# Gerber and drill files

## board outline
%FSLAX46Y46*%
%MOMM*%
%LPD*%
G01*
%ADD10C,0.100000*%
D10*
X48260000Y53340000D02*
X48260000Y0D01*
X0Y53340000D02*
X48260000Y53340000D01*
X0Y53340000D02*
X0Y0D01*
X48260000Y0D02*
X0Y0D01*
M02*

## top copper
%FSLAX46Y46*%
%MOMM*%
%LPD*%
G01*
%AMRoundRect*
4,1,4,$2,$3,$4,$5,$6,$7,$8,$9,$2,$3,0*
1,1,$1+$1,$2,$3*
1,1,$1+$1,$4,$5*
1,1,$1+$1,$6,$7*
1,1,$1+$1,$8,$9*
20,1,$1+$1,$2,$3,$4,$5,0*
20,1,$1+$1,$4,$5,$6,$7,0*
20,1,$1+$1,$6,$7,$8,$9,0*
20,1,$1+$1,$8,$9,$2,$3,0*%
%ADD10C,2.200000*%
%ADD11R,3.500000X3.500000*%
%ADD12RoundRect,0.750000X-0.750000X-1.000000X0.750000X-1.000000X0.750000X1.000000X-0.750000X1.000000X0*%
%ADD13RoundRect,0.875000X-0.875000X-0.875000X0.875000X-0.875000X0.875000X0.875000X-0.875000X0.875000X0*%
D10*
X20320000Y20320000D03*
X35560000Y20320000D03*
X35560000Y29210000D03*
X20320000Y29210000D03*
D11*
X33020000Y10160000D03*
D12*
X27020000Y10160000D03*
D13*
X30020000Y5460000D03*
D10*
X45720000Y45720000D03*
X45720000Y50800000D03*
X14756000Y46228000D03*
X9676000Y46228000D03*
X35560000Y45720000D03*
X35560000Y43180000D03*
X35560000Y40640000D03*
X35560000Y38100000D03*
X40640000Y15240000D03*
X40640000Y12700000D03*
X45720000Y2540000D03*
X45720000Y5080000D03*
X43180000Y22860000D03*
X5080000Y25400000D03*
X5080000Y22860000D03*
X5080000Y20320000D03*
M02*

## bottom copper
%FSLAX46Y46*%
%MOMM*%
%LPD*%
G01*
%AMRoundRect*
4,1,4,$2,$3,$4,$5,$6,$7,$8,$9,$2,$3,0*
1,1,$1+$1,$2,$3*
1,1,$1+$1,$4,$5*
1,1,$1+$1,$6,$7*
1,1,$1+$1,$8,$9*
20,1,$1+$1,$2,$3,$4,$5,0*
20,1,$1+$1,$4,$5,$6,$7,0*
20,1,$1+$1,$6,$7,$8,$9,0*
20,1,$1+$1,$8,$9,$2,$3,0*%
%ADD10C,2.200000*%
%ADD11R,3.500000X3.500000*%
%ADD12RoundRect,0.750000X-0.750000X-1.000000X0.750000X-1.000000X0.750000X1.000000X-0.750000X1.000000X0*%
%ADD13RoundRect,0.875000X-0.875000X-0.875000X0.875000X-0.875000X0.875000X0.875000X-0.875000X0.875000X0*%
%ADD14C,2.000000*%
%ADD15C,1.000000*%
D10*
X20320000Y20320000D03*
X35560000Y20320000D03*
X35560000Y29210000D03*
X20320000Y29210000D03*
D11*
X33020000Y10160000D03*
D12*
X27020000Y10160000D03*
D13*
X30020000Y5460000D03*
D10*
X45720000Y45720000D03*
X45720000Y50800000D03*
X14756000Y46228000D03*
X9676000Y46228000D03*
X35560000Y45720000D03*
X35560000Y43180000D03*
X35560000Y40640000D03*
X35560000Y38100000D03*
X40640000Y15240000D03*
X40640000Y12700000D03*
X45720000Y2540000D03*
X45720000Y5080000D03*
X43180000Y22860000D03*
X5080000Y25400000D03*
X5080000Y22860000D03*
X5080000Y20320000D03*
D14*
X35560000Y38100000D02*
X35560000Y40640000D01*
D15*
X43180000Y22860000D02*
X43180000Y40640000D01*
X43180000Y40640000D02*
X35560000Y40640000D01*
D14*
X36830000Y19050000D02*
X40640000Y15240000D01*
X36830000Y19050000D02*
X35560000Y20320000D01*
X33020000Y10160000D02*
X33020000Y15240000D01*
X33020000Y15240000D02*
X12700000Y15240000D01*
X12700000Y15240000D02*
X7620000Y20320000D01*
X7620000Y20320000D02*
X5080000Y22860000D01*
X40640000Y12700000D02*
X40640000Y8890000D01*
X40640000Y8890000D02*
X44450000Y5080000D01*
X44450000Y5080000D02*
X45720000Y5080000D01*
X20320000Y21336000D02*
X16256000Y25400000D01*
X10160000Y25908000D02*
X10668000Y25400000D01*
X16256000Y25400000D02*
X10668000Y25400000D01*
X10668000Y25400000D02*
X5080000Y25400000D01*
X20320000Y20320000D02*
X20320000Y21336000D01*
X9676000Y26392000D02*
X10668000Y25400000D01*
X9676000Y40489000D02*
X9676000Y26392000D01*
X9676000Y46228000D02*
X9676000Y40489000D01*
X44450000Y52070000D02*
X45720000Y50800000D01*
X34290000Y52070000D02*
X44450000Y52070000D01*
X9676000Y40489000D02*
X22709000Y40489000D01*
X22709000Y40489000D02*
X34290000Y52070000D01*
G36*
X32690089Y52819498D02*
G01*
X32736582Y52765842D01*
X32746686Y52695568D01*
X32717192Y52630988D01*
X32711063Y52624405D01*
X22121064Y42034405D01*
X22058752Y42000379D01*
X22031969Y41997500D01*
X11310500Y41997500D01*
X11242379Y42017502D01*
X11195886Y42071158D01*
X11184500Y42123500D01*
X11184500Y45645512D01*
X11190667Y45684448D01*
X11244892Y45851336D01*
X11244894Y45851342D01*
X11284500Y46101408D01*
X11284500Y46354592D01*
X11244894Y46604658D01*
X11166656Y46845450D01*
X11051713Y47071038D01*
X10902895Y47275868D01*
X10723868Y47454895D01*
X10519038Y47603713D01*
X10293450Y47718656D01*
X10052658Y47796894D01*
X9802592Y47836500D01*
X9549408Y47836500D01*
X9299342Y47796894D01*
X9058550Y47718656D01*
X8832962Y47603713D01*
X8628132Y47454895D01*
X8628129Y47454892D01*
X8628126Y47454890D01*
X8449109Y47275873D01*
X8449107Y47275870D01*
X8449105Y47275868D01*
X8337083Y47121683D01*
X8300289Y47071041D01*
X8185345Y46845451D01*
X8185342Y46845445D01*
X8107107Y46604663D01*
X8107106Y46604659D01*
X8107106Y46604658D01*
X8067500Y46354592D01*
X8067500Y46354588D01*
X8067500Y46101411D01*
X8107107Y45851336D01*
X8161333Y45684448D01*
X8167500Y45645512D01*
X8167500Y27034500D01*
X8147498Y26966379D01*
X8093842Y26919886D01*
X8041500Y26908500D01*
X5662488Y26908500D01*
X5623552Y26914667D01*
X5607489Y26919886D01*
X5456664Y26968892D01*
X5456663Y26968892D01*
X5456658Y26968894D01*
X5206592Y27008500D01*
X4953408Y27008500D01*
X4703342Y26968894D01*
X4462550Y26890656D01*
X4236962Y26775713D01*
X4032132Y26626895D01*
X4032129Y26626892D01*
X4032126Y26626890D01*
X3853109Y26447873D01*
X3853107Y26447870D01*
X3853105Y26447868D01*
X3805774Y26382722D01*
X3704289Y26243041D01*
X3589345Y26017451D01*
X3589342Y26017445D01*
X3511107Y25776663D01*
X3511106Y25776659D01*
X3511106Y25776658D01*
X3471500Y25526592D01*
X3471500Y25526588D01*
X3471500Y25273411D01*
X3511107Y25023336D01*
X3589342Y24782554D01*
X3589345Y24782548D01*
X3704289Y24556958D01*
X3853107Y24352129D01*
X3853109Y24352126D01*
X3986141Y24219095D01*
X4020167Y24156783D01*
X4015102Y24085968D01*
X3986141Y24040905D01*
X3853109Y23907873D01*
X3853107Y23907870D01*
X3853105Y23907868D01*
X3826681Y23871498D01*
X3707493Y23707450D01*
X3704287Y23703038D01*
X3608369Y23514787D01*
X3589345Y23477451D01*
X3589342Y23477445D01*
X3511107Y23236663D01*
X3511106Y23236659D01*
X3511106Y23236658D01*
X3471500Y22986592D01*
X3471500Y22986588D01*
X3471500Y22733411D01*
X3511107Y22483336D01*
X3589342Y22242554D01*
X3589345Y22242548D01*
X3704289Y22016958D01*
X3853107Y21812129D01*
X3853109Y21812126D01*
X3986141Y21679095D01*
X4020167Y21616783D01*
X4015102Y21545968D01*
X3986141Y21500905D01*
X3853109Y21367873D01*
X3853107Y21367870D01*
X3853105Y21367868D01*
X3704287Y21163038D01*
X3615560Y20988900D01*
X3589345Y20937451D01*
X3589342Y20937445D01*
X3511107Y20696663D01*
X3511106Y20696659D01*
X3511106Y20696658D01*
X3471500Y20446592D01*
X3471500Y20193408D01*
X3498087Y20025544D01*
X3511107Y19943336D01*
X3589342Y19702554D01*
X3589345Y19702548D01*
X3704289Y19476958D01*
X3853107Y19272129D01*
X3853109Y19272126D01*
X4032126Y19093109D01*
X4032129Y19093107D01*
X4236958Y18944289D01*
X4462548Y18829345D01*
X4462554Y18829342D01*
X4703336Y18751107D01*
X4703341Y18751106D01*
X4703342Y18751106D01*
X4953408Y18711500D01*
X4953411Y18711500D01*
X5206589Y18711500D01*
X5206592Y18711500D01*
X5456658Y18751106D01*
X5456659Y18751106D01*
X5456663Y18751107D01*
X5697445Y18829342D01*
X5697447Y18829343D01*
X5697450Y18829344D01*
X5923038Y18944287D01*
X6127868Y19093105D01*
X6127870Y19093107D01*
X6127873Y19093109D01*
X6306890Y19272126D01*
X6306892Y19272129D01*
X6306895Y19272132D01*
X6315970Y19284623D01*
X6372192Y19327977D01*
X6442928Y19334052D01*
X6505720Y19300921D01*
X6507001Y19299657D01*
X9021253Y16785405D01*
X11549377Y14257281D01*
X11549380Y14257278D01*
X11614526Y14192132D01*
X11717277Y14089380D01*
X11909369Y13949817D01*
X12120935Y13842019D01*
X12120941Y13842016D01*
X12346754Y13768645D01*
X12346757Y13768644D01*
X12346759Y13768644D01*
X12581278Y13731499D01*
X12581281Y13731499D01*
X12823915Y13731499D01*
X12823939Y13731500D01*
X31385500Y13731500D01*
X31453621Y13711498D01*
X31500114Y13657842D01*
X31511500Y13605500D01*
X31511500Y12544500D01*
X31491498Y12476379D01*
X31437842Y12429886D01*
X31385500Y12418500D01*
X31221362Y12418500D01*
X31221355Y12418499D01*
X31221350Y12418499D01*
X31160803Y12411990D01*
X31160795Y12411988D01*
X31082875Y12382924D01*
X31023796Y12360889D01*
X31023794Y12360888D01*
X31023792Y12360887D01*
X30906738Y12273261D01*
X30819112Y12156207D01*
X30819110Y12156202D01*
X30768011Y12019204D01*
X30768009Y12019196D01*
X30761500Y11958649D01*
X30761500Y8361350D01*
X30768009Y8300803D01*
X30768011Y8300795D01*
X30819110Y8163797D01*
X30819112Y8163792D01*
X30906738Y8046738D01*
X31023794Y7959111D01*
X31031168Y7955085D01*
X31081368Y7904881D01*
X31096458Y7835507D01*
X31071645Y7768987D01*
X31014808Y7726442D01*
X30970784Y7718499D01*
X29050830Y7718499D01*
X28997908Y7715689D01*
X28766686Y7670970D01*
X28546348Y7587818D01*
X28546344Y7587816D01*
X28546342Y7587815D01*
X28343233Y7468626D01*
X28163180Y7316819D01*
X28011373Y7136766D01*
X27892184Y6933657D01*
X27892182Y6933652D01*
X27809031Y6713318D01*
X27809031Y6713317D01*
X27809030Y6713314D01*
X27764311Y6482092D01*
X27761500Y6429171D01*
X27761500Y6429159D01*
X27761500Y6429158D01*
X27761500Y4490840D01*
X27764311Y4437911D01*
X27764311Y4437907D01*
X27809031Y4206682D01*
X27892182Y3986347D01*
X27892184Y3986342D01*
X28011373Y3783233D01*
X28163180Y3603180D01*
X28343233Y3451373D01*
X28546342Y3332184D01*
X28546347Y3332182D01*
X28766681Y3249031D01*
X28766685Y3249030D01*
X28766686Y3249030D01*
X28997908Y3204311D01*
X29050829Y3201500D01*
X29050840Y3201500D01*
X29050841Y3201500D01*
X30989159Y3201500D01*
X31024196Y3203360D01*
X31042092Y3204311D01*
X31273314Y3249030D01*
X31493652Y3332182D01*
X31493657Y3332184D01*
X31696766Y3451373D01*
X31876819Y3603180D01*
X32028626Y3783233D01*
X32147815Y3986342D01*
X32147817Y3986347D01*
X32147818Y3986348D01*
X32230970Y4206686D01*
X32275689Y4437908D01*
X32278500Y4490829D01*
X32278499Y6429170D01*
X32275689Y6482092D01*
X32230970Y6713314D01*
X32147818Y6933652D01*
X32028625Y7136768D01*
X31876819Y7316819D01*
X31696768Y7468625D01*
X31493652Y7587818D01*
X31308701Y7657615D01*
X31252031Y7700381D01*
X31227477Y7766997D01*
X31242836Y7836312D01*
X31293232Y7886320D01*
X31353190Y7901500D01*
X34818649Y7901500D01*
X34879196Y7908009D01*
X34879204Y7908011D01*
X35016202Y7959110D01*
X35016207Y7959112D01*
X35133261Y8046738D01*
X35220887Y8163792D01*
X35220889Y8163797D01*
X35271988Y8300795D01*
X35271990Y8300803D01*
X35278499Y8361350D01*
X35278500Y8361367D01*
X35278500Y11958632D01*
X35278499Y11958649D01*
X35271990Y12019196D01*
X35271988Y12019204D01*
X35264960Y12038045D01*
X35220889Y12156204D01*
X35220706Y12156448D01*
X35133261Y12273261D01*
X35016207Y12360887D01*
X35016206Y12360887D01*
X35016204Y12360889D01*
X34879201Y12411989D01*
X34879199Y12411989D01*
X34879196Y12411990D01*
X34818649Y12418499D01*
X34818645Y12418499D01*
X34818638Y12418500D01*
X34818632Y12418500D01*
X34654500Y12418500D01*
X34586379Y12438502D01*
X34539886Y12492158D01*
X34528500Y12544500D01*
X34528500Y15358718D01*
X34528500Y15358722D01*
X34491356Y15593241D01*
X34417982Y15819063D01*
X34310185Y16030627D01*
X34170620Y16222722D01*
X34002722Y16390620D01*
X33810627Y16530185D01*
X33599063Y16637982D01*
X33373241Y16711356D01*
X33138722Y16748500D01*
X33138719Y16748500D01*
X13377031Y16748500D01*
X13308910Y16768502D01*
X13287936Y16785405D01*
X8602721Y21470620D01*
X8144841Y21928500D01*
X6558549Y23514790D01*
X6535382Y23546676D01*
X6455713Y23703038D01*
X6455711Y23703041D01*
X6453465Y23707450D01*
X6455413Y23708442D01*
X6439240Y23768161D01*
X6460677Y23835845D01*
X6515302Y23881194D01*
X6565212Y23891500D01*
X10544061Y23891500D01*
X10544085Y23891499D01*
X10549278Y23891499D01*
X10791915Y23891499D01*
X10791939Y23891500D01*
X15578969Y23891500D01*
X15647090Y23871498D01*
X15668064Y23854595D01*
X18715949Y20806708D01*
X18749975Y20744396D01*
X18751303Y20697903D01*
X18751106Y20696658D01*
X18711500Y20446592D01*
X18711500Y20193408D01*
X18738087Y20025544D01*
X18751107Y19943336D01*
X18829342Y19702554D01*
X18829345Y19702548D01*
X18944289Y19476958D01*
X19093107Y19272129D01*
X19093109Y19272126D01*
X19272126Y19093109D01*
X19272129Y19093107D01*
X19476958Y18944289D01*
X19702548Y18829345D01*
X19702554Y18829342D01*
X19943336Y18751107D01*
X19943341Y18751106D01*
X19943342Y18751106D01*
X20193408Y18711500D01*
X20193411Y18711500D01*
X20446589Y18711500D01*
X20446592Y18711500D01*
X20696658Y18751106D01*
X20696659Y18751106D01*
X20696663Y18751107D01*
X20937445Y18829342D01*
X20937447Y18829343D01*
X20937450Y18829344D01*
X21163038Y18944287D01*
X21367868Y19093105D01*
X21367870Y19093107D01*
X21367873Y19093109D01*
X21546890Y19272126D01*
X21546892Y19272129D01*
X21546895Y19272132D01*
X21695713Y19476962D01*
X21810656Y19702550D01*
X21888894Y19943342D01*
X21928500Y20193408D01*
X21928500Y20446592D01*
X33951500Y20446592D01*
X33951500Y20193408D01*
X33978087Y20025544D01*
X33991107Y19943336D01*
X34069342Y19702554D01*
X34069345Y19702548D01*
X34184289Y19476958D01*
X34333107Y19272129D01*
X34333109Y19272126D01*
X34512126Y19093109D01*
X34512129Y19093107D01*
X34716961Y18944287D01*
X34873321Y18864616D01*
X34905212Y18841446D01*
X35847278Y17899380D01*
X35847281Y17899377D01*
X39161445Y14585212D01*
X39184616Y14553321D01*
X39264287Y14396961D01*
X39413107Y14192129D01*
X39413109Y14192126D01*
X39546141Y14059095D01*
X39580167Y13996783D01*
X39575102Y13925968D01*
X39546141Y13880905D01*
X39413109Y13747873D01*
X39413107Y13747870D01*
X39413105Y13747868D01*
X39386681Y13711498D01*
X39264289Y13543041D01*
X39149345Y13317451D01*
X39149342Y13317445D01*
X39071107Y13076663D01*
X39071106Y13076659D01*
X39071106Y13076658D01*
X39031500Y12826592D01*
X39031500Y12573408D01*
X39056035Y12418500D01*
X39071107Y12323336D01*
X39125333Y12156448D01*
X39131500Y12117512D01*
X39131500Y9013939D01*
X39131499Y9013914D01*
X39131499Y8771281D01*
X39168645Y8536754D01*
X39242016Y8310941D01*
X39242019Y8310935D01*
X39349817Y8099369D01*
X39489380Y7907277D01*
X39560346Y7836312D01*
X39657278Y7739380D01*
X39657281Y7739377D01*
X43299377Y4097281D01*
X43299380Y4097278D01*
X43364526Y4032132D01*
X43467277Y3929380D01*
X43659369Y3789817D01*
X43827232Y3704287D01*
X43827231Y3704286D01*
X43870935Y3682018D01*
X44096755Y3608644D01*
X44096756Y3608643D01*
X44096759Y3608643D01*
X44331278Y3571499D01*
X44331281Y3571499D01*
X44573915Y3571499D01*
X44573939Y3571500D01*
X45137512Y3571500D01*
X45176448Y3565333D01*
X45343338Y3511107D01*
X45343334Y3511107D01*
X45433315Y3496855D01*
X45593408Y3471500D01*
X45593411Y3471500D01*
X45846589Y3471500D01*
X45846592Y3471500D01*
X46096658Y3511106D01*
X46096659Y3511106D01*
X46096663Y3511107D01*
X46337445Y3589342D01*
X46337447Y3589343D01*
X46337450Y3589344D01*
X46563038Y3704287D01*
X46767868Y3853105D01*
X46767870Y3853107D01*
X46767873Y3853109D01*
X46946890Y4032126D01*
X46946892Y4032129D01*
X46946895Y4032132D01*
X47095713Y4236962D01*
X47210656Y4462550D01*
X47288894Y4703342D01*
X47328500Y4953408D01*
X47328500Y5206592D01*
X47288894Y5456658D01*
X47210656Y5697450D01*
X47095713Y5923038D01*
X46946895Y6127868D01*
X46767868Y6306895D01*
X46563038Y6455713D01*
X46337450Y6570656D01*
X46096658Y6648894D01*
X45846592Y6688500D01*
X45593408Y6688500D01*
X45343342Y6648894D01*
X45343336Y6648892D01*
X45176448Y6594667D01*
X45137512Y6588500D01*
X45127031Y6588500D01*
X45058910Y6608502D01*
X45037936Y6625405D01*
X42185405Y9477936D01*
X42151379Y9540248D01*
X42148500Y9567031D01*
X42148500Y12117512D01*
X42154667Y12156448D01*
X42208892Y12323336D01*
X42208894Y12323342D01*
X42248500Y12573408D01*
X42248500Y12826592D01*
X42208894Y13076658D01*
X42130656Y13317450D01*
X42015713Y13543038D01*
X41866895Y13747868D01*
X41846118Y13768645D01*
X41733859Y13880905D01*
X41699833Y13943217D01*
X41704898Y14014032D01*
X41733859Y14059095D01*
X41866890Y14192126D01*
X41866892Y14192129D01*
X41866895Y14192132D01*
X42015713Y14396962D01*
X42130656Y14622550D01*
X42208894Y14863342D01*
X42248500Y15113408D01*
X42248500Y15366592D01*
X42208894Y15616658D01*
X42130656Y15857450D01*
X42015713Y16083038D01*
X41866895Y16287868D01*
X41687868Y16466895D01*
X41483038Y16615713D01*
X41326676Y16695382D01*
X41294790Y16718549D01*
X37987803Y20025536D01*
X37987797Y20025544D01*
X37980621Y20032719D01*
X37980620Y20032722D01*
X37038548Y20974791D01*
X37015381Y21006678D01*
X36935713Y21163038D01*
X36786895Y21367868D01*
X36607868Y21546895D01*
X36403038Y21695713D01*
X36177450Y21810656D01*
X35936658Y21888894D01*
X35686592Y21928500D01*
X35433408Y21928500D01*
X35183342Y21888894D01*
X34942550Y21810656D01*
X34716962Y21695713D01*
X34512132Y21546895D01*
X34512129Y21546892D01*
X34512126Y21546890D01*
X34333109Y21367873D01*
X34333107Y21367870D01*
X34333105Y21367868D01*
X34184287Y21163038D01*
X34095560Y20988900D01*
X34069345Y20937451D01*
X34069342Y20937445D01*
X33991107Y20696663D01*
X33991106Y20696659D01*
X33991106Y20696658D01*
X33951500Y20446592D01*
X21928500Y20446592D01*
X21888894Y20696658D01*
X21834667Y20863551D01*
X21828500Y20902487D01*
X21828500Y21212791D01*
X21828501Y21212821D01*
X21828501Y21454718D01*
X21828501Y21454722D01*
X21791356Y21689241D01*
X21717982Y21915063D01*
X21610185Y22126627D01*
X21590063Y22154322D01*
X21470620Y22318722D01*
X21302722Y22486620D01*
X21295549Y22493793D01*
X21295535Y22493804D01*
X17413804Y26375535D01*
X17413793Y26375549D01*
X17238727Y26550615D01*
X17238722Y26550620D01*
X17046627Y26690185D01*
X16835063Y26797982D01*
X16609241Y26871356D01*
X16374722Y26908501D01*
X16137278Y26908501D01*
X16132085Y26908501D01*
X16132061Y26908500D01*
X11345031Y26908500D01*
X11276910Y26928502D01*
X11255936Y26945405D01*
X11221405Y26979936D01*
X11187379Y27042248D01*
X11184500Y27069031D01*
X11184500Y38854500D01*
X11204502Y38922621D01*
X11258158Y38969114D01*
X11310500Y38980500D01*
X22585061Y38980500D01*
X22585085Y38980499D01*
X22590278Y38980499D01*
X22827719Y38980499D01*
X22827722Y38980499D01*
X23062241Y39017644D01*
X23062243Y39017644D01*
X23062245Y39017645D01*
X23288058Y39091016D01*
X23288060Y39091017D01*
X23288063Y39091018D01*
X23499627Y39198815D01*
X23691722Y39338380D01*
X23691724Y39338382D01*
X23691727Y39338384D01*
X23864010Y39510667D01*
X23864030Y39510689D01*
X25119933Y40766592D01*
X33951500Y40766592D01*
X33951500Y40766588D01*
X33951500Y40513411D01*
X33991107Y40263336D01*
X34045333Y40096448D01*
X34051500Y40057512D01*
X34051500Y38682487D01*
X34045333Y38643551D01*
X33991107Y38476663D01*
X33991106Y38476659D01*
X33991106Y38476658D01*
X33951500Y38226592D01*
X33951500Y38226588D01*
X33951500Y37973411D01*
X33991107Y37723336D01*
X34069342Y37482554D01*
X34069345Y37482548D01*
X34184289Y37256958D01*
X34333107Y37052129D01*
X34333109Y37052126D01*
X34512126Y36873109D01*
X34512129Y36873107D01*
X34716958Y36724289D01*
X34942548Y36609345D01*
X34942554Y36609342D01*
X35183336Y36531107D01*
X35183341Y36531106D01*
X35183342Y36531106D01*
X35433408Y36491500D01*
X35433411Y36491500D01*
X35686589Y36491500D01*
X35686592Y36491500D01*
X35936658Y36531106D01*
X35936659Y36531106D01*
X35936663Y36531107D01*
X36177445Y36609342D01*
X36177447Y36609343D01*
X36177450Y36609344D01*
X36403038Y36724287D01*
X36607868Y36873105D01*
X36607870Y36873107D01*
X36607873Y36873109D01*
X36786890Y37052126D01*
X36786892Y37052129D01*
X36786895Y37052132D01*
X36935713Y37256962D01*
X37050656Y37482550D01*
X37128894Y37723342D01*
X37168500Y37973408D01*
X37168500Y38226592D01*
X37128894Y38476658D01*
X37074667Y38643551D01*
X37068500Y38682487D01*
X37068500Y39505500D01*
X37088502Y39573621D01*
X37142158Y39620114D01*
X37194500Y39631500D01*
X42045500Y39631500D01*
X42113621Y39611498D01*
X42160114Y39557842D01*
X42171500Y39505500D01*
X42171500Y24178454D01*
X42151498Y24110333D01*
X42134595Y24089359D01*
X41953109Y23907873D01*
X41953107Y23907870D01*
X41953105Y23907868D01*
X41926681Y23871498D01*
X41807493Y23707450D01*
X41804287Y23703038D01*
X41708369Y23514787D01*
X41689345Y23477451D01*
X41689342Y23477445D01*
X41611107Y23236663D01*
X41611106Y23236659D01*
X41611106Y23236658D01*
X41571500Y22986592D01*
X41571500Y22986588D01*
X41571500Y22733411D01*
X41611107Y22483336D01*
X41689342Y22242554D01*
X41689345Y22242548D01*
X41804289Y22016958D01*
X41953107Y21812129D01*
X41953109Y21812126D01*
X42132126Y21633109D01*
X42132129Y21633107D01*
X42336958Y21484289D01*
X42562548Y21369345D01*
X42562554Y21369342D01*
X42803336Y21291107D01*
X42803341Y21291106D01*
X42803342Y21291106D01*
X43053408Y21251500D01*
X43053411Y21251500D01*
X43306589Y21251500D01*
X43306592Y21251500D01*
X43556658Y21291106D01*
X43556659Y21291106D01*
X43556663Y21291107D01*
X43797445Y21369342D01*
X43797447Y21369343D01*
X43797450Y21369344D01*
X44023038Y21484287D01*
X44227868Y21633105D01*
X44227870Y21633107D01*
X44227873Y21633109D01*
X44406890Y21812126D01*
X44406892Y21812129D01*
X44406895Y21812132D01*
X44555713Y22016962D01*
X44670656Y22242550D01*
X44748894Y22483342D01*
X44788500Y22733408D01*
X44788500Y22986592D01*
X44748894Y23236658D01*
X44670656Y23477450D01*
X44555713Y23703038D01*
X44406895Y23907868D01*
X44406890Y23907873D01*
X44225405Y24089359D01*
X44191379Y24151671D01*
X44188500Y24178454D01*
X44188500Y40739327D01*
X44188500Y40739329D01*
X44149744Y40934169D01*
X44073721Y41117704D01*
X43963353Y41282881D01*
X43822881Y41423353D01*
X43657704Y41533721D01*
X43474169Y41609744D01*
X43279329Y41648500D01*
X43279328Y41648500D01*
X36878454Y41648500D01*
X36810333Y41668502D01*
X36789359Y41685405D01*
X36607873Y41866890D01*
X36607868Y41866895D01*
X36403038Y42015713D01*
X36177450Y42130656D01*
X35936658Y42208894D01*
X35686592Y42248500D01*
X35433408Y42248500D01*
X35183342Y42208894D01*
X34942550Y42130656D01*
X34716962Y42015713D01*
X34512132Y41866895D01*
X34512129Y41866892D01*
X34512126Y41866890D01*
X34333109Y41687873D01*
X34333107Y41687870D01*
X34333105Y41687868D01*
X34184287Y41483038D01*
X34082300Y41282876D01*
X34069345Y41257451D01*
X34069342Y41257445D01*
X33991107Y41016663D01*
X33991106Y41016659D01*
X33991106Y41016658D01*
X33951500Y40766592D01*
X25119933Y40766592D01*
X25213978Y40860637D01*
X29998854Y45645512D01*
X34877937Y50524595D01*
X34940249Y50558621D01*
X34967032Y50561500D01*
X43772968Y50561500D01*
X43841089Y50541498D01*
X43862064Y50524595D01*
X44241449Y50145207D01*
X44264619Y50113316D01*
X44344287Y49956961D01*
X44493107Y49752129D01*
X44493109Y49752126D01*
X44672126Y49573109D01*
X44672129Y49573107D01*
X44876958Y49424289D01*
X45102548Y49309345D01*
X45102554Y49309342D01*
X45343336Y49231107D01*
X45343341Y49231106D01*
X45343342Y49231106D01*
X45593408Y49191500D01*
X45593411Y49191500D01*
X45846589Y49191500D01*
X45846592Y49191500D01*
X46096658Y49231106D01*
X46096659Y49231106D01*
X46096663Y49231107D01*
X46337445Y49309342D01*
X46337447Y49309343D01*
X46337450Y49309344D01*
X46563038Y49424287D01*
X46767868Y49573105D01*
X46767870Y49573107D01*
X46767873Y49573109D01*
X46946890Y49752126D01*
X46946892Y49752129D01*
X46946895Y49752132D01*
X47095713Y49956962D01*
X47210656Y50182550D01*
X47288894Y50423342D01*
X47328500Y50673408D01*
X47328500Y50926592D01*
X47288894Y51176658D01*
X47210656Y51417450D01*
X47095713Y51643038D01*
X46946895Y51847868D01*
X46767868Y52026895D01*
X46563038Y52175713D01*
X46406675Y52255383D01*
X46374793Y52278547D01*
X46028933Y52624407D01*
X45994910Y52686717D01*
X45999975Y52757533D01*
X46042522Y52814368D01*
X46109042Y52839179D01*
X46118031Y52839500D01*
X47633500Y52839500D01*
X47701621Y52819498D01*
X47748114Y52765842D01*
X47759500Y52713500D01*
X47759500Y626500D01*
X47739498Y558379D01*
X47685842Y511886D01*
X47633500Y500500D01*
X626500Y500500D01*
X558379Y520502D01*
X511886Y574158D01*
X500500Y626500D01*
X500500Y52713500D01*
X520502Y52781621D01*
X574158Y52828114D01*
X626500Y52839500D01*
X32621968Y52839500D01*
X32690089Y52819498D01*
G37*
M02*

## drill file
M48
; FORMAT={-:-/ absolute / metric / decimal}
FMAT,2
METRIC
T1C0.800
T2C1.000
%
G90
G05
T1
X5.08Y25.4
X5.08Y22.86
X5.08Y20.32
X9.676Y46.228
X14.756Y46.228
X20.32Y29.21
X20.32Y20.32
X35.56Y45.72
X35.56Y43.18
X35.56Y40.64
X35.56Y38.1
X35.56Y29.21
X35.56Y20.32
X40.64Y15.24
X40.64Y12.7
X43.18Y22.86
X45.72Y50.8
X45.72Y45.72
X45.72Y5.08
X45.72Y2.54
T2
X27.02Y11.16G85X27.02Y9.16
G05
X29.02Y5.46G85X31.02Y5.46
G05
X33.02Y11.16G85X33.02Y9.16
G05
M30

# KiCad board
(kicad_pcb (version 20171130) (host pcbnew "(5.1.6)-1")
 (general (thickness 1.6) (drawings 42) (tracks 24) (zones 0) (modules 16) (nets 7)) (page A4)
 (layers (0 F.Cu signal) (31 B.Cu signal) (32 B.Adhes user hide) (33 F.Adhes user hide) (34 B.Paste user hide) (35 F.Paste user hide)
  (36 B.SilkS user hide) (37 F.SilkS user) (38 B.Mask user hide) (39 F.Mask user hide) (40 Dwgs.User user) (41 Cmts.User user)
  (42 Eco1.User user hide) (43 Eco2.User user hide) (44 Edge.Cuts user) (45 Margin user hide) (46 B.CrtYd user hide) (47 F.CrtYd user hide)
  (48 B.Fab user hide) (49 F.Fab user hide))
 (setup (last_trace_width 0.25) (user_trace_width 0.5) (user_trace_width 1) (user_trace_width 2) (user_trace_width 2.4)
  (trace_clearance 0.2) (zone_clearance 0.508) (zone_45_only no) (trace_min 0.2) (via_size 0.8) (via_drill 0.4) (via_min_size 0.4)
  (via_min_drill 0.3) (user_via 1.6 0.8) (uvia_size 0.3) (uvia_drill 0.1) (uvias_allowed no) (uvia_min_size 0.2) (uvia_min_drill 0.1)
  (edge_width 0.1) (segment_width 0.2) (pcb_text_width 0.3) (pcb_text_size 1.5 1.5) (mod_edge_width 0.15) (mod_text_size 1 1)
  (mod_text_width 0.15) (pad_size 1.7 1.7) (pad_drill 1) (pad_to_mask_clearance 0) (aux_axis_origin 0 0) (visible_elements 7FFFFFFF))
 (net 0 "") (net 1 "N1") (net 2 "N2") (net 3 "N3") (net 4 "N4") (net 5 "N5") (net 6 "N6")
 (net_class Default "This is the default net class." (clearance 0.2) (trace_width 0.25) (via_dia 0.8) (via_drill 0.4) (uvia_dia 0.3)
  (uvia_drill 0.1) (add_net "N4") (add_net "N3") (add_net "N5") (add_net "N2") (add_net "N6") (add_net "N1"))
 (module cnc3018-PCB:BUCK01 (layer F.Cu) (at 25.4 -29.21)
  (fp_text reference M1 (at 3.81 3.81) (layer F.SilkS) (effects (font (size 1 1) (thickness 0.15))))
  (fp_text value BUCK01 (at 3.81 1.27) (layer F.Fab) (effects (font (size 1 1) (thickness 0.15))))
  (pad 4 thru_hole circle (at -5.08 8.89) (size 2.2 2.2) (drill 0.8) (layers *.Cu *.Mask) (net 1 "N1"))
  (pad 3 thru_hole circle (at 10.16 8.89) (size 2.2 2.2) (drill 0.8) (layers *.Cu *.Mask) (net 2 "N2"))
  (pad 2 thru_hole circle (at 10.16 0) (size 2.2 2.2) (drill 0.8) (layers *.Cu *.Mask) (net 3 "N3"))
  (pad 1 thru_hole circle (at -5.08 0) (size 2.2 2.2) (drill 0.8) (layers *.Cu *.Mask) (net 3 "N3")))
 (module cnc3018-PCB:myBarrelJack (layer F.Cu) (at 33.02 -10.16)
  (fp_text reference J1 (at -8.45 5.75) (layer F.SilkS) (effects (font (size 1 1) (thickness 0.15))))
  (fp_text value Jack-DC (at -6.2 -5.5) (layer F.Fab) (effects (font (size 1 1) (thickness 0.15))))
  (pad 1 thru_hole rect (at 0 0) (size 3.5 3.5) (drill oval 1 3) (layers *.Cu *.Mask) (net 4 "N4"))
  (pad 2 thru_hole roundrect (at -6 0) (size 3 3.5) (drill oval 1 3) (layers *.Cu *.Mask) (roundrect_rratio 0.25) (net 3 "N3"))
  (pad 3 thru_hole roundrect (at -3 4.7) (size 3.5 3.5) (drill oval 3 1) (layers *.Cu *.Mask) (roundrect_rratio 0.25)))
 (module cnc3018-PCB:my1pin (layer F.Cu) (at 45.72 -45.72)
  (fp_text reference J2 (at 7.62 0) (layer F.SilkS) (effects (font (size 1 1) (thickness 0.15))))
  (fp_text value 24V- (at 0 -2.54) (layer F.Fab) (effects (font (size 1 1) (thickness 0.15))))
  (pad 1 thru_hole circle (at 0 0) (size 2.2 2.2) (drill 0.8) (layers *.Cu *.Mask) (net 3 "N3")))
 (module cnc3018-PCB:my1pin (layer F.Cu) (at 45.72 -50.8)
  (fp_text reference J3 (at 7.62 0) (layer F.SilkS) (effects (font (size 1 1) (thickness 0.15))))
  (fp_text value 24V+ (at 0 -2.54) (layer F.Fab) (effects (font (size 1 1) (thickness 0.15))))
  (pad 1 thru_hole circle (at 0 0) (size 2.2 2.2) (drill 0.8) (layers *.Cu *.Mask) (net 1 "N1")))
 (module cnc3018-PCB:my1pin (layer F.Cu) (at 14.756 -46.228 180)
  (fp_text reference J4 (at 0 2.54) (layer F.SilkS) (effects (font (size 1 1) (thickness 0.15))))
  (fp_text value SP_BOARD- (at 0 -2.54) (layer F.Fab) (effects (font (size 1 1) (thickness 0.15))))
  (pad 1 thru_hole circle (at 0 0 180) (size 2.2 2.2) (drill 0.8) (layers *.Cu *.Mask) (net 3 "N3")))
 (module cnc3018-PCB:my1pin (layer F.Cu) (at 9.676 -46.228 180)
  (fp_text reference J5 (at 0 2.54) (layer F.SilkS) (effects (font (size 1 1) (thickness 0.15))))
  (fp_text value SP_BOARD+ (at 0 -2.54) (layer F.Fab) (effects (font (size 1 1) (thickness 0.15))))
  (pad 1 thru_hole circle (at 0 0 180) (size 2.2 2.2) (drill 0.8) (layers *.Cu *.Mask) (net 1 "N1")))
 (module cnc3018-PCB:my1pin (layer F.Cu) (at 35.56 -45.72 180)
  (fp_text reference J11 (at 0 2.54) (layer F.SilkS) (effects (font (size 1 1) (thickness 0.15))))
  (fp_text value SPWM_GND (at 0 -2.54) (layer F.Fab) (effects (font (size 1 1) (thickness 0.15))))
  (pad 1 thru_hole circle (at 0 0 180) (size 2.2 2.2) (drill 0.8) (layers *.Cu *.Mask) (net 3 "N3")))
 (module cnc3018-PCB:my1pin (layer F.Cu) (at 35.56 -43.18 180)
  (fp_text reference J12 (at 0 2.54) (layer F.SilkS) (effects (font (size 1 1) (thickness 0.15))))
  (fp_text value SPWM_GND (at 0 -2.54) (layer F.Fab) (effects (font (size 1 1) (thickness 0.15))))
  (pad 1 thru_hole circle (at 0 0 180) (size 2.2 2.2) (drill 0.8) (layers *.Cu *.Mask) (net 3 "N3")))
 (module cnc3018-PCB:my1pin (layer F.Cu) (at 35.56 -40.64 180)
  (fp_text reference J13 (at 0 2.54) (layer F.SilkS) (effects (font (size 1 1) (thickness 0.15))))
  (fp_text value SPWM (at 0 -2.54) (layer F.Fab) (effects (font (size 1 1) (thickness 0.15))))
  (pad 1 thru_hole circle (at 0 0 180) (size 2.2 2.2) (drill 0.8) (layers *.Cu *.Mask) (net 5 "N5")))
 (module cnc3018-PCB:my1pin (layer F.Cu) (at 35.56 -38.1 180)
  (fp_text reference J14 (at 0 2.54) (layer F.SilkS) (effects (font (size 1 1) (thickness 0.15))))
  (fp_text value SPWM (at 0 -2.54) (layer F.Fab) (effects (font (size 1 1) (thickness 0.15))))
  (pad 1 thru_hole circle (at 0 0 180) (size 2.2 2.2) (drill 0.8) (layers *.Cu *.Mask) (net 5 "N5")))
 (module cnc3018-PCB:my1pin (layer F.Cu) (at 40.64 -15.24 270)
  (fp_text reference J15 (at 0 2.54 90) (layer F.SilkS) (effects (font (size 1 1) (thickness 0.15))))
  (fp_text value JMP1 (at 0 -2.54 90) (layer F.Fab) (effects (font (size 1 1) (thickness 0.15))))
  (pad 1 thru_hole circle (at 0 0 270) (size 2.2 2.2) (drill 0.8) (layers *.Cu *.Mask) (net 2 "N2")))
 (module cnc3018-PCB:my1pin (layer F.Cu) (at 40.64 -12.7 270)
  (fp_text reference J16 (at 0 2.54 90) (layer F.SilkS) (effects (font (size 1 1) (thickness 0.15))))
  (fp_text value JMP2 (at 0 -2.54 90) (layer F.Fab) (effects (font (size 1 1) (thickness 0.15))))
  (pad 1 thru_hole circle (at 0 0 270) (size 2.2 2.2) (drill 0.8) (layers *.Cu *.Mask) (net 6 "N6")))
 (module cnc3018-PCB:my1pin (layer F.Cu) (at 45.72 -2.54)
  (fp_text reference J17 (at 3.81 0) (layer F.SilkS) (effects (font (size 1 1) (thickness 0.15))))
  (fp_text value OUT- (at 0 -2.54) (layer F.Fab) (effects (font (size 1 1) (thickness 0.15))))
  (pad 1 thru_hole circle (at 0 0) (size 2.2 2.2) (drill 0.8) (layers *.Cu *.Mask) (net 3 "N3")))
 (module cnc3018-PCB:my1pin (layer F.Cu) (at 45.72 -5.08)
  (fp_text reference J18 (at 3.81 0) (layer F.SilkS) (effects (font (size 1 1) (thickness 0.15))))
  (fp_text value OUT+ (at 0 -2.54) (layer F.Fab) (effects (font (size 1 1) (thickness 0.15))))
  (pad 1 thru_hole circle (at 0 0) (size 2.2 2.2) (drill 0.8) (layers *.Cu *.Mask) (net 6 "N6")))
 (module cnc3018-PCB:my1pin (layer F.Cu) (at 43.18 -22.86)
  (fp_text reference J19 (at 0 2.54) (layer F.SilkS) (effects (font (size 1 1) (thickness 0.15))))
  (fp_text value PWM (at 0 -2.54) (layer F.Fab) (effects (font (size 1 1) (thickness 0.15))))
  (pad 1 thru_hole circle (at 0 0) (size 2.2 2.2) (drill 0.8) (layers *.Cu *.Mask) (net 5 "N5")))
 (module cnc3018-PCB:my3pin (layer F.Cu) (at 5.08 -22.86 270)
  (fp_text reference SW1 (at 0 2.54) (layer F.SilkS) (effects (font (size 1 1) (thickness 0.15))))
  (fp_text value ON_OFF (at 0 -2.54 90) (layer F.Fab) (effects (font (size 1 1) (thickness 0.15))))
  (pad 1 thru_hole circle (at -2.54 0 270) (size 2.2 2.2) (drill 0.8) (layers *.Cu *.Mask) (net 1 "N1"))
  (pad 2 thru_hole circle (at 0 0 270) (size 2.2 2.2) (drill 0.8) (layers *.Cu *.Mask) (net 4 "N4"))
  (pad 3 thru_hole circle (at 2.54 0 270) (size 2.2 2.2) (drill 0.8) (layers *.Cu *.Mask)))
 (gr_line (start 48.26 -53.34) (end 48.26 0) (layer Edge.Cuts) (width 0.1))
 (gr_line (start 0 -53.34) (end 48.26 -53.34) (layer Edge.Cuts) (width 0.1))
 (gr_line (start 0 -53.34) (end 0 0) (layer Edge.Cuts) (width 0.1))
 (gr_line (start 48.26 0) (end 0 0) (layer Edge.Cuts) (width 0.1))
 (segment (start 35.56 -38.1) (end 35.56 -40.64) (width 2) (layer B.Cu) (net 5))
 (segment (start 43.18 -22.86) (end 43.18 -40.64) (width 1) (layer B.Cu) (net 5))
 (segment (start 43.18 -40.64) (end 35.56 -40.64) (width 1) (layer B.Cu) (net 5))
 (segment (start 36.83 -19.05) (end 40.64 -15.24) (width 2) (layer B.Cu) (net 2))
 (segment (start 36.83 -19.05) (end 35.56 -20.32) (width 2) (layer B.Cu) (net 2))
 (segment (start 33.02 -10.16) (end 33.02 -15.24) (width 2) (layer B.Cu) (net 4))
 (segment (start 33.02 -15.24) (end 12.7 -15.24) (width 2) (layer B.Cu) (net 4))
 (segment (start 12.7 -15.24) (end 7.62 -20.32) (width 2) (layer B.Cu) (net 4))
 (segment (start 7.62 -20.32) (end 5.08 -22.86) (width 2) (layer B.Cu) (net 4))
 (segment (start 40.64 -12.7) (end 40.64 -8.89) (width 2) (layer B.Cu) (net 6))
 (segment (start 40.64 -8.89) (end 44.45 -5.08) (width 2) (layer B.Cu) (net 6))
 (segment (start 44.45 -5.08) (end 45.72 -5.08) (width 2) (layer B.Cu) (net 6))
 (segment (start 20.32 -21.336) (end 16.256 -25.4) (width 2) (layer B.Cu) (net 1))
 (segment (start 10.16 -25.908) (end 10.668 -25.4) (width 2) (layer B.Cu) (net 1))
 (segment (start 16.256 -25.4) (end 10.668 -25.4) (width 2) (layer B.Cu) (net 1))
 (segment (start 10.668 -25.4) (end 5.08 -25.4) (width 2) (layer B.Cu) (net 1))
 (segment (start 20.32 -20.32) (end 20.32 -21.336) (width 2) (layer B.Cu) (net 1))
 (segment (start 9.676 -26.392) (end 10.668 -25.4) (width 2) (layer B.Cu) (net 1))
 (segment (start 9.676 -40.489) (end 9.676 -26.392) (width 2) (layer B.Cu) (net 1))
 (segment (start 9.676 -46.228) (end 9.676 -40.489) (width 2) (layer B.Cu) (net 1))
 (segment (start 44.45 -52.07) (end 45.72 -50.8) (width 2) (layer B.Cu) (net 1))
 (segment (start 34.29 -52.07) (end 44.45 -52.07) (width 2) (layer B.Cu) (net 1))
 (segment (start 9.676 -40.489) (end 22.709 -40.489) (width 2) (layer B.Cu) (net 1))
 (segment (start 22.709 -40.489) (end 34.29 -52.07) (width 2) (layer B.Cu) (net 1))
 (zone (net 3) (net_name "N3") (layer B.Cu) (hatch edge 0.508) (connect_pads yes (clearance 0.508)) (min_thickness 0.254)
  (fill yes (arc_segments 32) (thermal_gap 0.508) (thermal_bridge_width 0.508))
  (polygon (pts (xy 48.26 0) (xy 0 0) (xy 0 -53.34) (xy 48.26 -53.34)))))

